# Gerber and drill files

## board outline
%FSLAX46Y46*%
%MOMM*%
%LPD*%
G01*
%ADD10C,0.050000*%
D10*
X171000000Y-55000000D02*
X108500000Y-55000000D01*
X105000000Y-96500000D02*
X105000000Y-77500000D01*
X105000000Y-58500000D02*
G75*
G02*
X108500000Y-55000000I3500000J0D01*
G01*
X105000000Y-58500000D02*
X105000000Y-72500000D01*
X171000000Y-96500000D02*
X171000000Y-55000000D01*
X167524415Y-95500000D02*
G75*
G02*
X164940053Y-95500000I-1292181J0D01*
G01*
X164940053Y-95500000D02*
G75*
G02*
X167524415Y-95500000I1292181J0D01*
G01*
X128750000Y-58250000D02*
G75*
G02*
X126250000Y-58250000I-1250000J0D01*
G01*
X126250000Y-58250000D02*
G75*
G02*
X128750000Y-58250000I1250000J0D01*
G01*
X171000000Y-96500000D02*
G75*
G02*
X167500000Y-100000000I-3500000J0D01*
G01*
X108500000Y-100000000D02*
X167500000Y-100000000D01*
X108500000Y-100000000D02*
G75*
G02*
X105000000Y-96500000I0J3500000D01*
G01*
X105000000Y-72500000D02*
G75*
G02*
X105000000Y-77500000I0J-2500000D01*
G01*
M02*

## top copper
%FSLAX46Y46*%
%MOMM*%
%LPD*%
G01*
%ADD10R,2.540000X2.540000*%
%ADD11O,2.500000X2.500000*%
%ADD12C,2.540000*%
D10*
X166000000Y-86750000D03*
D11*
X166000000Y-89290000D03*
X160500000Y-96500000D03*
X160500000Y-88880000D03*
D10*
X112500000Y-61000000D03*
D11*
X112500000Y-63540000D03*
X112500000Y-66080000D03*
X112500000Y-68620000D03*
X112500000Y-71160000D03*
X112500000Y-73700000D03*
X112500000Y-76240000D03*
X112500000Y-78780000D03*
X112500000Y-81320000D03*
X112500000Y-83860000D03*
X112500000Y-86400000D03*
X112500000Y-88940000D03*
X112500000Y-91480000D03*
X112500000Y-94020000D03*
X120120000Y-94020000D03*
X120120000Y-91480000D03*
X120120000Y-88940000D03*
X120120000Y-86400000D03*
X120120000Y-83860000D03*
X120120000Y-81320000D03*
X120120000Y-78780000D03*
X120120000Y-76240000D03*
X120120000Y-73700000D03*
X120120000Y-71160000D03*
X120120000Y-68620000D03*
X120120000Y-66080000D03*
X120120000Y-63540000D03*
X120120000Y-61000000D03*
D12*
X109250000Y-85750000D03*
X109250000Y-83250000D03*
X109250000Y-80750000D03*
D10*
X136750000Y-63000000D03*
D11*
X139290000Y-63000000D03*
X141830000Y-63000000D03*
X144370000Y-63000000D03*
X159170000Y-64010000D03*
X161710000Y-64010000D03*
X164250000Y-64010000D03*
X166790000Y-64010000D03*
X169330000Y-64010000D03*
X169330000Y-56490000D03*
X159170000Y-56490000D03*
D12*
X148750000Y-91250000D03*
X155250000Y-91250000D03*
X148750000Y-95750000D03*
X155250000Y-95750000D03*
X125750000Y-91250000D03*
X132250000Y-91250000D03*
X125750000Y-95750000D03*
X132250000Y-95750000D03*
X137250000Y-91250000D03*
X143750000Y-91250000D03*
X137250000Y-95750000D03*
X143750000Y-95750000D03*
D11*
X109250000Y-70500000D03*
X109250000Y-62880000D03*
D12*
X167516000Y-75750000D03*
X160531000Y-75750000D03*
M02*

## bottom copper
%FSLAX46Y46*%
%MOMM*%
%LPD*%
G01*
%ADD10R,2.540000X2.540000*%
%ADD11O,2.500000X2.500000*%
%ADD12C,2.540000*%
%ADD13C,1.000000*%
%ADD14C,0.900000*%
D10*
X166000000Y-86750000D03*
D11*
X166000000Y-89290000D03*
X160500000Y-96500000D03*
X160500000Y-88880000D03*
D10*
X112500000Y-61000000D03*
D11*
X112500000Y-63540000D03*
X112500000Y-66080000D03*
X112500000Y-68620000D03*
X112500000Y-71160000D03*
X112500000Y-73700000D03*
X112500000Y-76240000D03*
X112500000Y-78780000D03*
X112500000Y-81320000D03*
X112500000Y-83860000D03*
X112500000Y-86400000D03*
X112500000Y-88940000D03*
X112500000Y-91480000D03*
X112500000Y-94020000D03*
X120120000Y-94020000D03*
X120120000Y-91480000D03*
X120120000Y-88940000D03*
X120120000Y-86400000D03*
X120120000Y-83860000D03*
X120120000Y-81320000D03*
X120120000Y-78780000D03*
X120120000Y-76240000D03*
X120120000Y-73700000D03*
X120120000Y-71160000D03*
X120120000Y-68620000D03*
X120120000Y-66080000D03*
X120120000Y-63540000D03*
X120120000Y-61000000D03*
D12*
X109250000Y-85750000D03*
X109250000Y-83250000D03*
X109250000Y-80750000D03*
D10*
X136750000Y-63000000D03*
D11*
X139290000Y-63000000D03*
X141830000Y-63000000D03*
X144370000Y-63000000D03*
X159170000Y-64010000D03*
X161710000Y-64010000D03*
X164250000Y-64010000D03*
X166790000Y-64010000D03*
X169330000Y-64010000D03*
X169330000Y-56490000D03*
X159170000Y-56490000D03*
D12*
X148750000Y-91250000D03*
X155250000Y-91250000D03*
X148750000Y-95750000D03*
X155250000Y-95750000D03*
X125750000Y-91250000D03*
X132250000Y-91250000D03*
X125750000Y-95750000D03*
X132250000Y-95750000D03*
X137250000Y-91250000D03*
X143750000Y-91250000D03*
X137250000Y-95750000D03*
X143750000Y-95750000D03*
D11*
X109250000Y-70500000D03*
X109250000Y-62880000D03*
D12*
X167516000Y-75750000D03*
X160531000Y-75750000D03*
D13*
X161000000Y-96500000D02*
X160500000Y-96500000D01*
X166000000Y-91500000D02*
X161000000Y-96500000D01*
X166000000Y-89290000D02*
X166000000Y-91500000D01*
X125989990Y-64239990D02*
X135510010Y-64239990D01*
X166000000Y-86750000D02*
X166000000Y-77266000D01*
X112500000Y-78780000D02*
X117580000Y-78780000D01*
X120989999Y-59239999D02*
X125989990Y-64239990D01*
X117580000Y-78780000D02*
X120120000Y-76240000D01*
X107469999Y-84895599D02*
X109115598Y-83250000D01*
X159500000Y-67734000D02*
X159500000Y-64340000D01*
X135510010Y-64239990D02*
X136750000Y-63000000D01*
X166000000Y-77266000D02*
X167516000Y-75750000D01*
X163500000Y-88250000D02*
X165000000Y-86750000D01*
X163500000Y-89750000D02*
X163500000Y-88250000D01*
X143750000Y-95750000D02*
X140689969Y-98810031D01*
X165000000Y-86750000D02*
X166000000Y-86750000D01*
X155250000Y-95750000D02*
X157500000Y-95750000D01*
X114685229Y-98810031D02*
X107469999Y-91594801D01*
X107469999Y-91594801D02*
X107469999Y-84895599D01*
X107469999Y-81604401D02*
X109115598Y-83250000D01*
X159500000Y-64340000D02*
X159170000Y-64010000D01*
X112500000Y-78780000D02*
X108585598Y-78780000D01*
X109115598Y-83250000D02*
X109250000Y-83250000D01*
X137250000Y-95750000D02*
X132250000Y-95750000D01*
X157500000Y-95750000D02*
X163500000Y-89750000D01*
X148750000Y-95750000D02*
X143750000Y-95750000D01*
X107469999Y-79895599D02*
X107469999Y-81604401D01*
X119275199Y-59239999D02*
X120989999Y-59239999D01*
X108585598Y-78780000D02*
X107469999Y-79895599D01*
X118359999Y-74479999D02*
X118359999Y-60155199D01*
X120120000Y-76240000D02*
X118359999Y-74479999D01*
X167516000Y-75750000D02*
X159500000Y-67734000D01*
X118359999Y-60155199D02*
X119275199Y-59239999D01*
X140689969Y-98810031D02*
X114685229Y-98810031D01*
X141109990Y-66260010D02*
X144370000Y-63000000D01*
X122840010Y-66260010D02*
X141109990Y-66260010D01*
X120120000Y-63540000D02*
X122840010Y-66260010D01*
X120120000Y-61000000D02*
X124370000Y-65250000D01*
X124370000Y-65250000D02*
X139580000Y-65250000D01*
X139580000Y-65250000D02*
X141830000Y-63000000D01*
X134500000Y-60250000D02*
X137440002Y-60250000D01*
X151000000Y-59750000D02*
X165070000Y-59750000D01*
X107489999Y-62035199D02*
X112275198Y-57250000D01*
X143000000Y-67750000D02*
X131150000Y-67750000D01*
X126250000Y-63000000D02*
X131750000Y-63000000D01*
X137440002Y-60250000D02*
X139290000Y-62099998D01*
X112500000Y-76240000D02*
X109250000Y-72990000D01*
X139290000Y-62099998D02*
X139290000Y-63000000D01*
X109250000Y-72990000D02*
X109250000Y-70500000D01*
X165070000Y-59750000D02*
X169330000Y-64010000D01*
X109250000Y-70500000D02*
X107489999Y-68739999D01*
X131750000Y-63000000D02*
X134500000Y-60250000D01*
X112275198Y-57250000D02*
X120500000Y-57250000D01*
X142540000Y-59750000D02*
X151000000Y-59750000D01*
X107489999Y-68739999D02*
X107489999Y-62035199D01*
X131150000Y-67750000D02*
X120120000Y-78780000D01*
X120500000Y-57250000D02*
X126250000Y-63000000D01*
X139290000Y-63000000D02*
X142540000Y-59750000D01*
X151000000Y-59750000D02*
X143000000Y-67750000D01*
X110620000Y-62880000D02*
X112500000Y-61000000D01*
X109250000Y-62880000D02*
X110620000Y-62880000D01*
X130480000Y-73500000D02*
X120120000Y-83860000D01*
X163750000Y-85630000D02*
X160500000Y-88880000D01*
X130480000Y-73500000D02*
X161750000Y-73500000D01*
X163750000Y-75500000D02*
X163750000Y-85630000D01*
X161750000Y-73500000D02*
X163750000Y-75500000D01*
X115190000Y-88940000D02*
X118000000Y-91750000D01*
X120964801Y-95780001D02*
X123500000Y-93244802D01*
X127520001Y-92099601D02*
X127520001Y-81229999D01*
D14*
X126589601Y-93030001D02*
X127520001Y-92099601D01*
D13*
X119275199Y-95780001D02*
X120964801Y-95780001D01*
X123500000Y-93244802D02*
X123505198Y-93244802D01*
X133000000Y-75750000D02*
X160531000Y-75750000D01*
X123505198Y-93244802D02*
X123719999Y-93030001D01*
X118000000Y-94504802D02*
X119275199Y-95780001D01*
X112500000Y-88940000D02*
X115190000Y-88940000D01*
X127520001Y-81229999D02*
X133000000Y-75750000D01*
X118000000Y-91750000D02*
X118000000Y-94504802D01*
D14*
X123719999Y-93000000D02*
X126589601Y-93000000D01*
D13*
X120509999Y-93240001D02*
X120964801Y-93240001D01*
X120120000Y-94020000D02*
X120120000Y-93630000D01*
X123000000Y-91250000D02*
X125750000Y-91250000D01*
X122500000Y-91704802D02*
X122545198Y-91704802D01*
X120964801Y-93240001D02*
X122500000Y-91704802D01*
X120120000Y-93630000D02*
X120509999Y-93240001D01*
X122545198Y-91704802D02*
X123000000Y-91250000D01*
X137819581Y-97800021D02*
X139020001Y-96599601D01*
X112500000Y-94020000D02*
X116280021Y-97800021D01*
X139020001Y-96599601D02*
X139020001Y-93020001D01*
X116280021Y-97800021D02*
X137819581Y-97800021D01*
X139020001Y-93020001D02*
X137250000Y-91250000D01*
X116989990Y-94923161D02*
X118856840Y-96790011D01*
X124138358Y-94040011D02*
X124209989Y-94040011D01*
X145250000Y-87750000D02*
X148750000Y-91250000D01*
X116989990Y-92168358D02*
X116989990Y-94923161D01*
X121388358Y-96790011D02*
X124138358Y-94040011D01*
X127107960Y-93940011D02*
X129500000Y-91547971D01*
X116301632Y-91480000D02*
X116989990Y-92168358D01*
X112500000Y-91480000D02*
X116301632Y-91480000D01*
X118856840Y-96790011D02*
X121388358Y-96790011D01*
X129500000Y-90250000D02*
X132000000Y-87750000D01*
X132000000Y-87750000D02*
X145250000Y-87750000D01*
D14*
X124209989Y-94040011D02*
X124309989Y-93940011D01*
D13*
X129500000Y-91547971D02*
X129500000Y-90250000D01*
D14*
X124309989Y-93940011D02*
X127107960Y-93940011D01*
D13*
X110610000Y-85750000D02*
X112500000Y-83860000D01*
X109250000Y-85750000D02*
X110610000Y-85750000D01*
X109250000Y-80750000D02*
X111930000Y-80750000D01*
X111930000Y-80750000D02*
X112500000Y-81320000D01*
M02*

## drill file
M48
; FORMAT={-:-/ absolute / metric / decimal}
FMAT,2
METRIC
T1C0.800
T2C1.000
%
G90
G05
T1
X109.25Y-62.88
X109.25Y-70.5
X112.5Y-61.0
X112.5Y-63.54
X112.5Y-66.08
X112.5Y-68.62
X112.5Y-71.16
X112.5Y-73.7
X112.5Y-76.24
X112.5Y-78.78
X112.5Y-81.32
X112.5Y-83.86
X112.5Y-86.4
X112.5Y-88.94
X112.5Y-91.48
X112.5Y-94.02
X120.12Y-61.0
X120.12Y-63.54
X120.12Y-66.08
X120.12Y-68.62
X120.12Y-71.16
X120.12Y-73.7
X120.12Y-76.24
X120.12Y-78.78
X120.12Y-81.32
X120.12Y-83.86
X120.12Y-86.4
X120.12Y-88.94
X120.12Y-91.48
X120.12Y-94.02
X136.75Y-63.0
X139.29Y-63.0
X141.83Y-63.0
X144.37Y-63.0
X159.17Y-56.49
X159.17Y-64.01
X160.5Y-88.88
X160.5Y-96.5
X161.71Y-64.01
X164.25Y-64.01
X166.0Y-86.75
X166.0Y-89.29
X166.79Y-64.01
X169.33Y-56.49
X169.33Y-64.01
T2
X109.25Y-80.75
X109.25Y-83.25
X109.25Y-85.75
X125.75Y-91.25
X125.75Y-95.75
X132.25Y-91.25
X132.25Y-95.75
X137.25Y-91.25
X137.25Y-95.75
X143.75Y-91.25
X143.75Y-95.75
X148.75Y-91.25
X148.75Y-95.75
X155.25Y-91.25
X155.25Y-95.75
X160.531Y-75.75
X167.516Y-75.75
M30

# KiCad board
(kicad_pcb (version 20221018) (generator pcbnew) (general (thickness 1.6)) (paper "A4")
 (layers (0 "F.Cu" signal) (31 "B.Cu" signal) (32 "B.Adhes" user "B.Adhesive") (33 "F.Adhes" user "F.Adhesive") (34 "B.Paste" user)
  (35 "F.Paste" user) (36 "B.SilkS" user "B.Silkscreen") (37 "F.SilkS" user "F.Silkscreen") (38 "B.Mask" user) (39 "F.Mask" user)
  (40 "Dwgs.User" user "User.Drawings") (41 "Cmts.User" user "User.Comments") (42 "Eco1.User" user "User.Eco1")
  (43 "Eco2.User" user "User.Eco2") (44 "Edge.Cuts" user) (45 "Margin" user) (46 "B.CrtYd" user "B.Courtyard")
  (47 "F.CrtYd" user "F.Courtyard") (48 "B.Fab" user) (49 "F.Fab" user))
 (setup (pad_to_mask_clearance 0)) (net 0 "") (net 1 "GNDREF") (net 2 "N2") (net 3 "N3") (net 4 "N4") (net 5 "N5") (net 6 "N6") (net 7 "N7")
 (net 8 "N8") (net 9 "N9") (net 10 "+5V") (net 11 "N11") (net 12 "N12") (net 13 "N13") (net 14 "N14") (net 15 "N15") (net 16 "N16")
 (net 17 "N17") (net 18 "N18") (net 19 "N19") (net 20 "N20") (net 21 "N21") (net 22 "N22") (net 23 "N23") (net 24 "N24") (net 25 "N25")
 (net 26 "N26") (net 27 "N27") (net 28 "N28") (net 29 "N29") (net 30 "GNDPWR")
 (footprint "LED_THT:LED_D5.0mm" (layer "F.Cu") (at 166 86.75 -90)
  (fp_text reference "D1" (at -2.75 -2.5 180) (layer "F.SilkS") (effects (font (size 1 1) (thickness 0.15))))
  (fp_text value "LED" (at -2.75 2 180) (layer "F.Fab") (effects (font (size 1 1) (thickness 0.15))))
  (pad "1" thru_hole rect (at 0 0 270) (size 2.54 2.54) (drill 0.8) (layers "*.Cu" "*.Mask") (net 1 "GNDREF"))
  (pad "2" thru_hole oval (at 2.54 0 270) (size 2.5 2.5) (drill 0.8) (layers "*.Cu" "*.Mask") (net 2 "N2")))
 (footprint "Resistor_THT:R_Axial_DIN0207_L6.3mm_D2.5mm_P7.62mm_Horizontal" (layer "F.Cu") (at 160.5 96.5 90)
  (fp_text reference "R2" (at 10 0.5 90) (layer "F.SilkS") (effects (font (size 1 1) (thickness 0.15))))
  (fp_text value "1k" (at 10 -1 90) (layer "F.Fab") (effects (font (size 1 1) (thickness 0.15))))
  (pad "1" thru_hole oval (at 0 0 90) (size 2.5 2.5) (drill 0.8) (layers "*.Cu" "*.Mask") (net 2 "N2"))
  (pad "2" thru_hole oval (at 7.62 0 90) (size 2.5 2.5) (drill 0.8) (layers "*.Cu" "*.Mask") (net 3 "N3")))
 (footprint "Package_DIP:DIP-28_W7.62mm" (layer "F.Cu") (at 112.5 61)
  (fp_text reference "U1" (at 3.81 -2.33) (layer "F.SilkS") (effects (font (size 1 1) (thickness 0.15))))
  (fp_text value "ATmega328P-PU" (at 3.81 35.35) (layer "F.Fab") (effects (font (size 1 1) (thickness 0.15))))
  (pad "1" thru_hole rect (at 0 0) (size 2.54 2.54) (drill 0.8) (layers "*.Cu" "*.Mask") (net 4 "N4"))
  (pad "2" thru_hole oval (at 0 2.54) (size 2.5 2.5) (drill 0.8) (layers "*.Cu" "*.Mask") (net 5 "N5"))
  (pad "3" thru_hole oval (at 0 5.08) (size 2.5 2.5) (drill 0.8) (layers "*.Cu" "*.Mask") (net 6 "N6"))
  (pad "4" thru_hole oval (at 0 7.62) (size 2.5 2.5) (drill 0.8) (layers "*.Cu" "*.Mask") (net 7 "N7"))
  (pad "5" thru_hole oval (at 0 10.16) (size 2.5 2.5) (drill 0.8) (layers "*.Cu" "*.Mask") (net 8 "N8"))
  (pad "6" thru_hole oval (at 0 12.7) (size 2.5 2.5) (drill 0.8) (layers "*.Cu" "*.Mask") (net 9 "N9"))
  (pad "7" thru_hole oval (at 0 15.24) (size 2.5 2.5) (drill 0.8) (layers "*.Cu" "*.Mask") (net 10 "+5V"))
  (pad "8" thru_hole oval (at 0 17.78) (size 2.5 2.5) (drill 0.8) (layers "*.Cu" "*.Mask") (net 1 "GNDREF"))
  (pad "9" thru_hole oval (at 0 20.32) (size 2.5 2.5) (drill 0.8) (layers "*.Cu" "*.Mask") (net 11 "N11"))
  (pad "10" thru_hole oval (at 0 22.86) (size 2.5 2.5) (drill 0.8) (layers "*.Cu" "*.Mask") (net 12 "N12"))
  (pad "11" thru_hole oval (at 0 25.4) (size 2.5 2.5) (drill 0.8) (layers "*.Cu" "*.Mask") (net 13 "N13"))
  (pad "12" thru_hole oval (at 0 27.94) (size 2.5 2.5) (drill 0.8) (layers "*.Cu" "*.Mask") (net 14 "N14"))
  (pad "13" thru_hole oval (at 0 30.48) (size 2.5 2.5) (drill 0.8) (layers "*.Cu" "*.Mask") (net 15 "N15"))
  (pad "14" thru_hole oval (at 0 33.02) (size 2.5 2.5) (drill 0.8) (layers "*.Cu" "*.Mask") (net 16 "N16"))
  (pad "15" thru_hole oval (at 7.62 33.02) (size 2.5 2.5) (drill 0.8) (layers "*.Cu" "*.Mask") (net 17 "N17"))
  (pad "16" thru_hole oval (at 7.62 30.48) (size 2.5 2.5) (drill 0.8) (layers "*.Cu" "*.Mask") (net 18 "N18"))
  (pad "17" thru_hole oval (at 7.62 27.94) (size 2.5 2.5) (drill 0.8) (layers "*.Cu" "*.Mask") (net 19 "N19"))
  (pad "18" thru_hole oval (at 7.62 25.4) (size 2.5 2.5) (drill 0.8) (layers "*.Cu" "*.Mask") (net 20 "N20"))
  (pad "19" thru_hole oval (at 7.62 22.86) (size 2.5 2.5) (drill 0.8) (layers "*.Cu" "*.Mask") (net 3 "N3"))
  (pad "20" thru_hole oval (at 7.62 20.32) (size 2.5 2.5) (drill 0.8) (layers "*.Cu" "*.Mask") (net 10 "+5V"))
  (pad "21" thru_hole oval (at 7.62 17.78) (size 2.5 2.5) (drill 0.8) (layers "*.Cu" "*.Mask") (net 10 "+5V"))
  (pad "22" thru_hole oval (at 7.62 15.24) (size 2.5 2.5) (drill 0.8) (layers "*.Cu" "*.Mask") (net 1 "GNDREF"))
  (pad "23" thru_hole oval (at 7.62 12.7) (size 2.5 2.5) (drill 0.8) (layers "*.Cu" "*.Mask") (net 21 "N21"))
  (pad "24" thru_hole oval (at 7.62 10.16) (size 2.5 2.5) (drill 0.8) (layers "*.Cu" "*.Mask") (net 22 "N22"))
  (pad "25" thru_hole oval (at 7.62 7.62) (size 2.5 2.5) (drill 0.8) (layers "*.Cu" "*.Mask") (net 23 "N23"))
  (pad "26" thru_hole oval (at 7.62 5.08) (size 2.5 2.5) (drill 0.8) (layers "*.Cu" "*.Mask") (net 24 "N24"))
  (pad "27" thru_hole oval (at 7.62 2.54) (size 2.5 2.5) (drill 0.8) (layers "*.Cu" "*.Mask") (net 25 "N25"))
  (pad "28" thru_hole oval (at 7.62 0) (size 2.5 2.5) (drill 0.8) (layers "*.Cu" "*.Mask") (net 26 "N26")))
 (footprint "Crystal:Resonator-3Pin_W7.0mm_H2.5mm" (layer "F.Cu") (at 109.25 85.75 90)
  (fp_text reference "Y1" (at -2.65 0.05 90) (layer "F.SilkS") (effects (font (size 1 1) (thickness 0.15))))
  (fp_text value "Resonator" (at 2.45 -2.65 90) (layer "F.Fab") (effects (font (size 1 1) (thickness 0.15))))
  (pad "1" thru_hole circle (at 0 0 90) (size 2.54 2.54) (drill 1) (layers "*.Cu" "*.Mask") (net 12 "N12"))
  (pad "2" thru_hole circle (at 2.5 0 90) (size 2.54 2.54) (drill 1) (layers "*.Cu" "*.Mask") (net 1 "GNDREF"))
  (pad "3" thru_hole circle (at 5 0 90) (size 2.54 2.54) (drill 1) (layers "*.Cu" "*.Mask") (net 11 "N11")))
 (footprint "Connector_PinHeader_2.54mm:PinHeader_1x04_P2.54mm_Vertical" (layer "F.Cu") (at 136.75 63 90)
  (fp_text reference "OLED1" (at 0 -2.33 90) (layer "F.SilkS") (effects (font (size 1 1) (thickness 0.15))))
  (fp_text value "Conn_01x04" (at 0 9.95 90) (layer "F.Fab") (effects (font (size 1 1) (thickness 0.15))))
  (pad "1" thru_hole rect (at 0 0 90) (size 2.54 2.54) (drill 0.8) (layers "*.Cu" "*.Mask") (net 1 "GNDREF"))
  (pad "2" thru_hole oval (at 0 2.54 90) (size 2.5 2.5) (drill 0.8) (layers "*.Cu" "*.Mask") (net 10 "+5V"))
  (pad "3" thru_hole oval (at 0 5.08 90) (size 2.5 2.5) (drill 0.8) (layers "*.Cu" "*.Mask") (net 26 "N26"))
  (pad "4" thru_hole oval (at 0 7.62 90) (size 2.5 2.5) (drill 0.8) (layers "*.Cu" "*.Mask") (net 25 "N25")))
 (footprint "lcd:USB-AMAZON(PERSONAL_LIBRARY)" (layer "F.Cu") (at 164.25 60.25)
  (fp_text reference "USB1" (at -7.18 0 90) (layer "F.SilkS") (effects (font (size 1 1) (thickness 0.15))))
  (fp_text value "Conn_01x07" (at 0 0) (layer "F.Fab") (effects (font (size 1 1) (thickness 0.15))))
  (pad "1" thru_hole oval (at -5.08 3.76) (size 2.5 2.5) (drill 0.8) (layers "*.Cu" "*.Mask") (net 1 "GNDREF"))
  (pad "2" thru_hole oval (at -2.54 3.76) (size 2.5 2.5) (drill 0.8) (layers "*.Cu" "*.Mask") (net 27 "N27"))
  (pad "3" thru_hole oval (at 0 3.76) (size 2.5 2.5) (drill 0.8) (layers "*.Cu" "*.Mask") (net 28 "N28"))
  (pad "4" thru_hole oval (at 2.54 3.76) (size 2.5 2.5) (drill 0.8) (layers "*.Cu" "*.Mask") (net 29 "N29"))
  (pad "5" thru_hole oval (at 5.08 3.76) (size 2.5 2.5) (drill 0.8) (layers "*.Cu" "*.Mask") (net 10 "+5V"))
  (pad "6" thru_hole oval (at 5.08 -3.76) (size 2.5 2.5) (drill 0.8) (layers "*.Cu" "*.Mask") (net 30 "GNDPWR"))
  (pad "7" thru_hole oval (at -5.08 -3.76) (size 2.5 2.5) (drill 0.8) (layers "*.Cu" "*.Mask") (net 30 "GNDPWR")))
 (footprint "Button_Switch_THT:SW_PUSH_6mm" (layer "F.Cu") (at 148.75 91.25)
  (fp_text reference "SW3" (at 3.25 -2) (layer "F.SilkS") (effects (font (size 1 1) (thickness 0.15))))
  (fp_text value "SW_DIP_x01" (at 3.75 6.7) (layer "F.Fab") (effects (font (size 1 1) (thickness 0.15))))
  (pad "1" thru_hole circle (at 0 0) (size 2.54 2.54) (drill 1) (layers "*.Cu" "*.Mask") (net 15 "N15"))
  (pad "1" thru_hole circle (at 6.5 0) (size 2.54 2.54) (drill 1) (layers "*.Cu" "*.Mask") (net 15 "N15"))
  (pad "2" thru_hole circle (at 0 4.5) (size 2.54 2.54) (drill 1) (layers "*.Cu" "*.Mask") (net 1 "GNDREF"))
  (pad "2" thru_hole circle (at 6.5 4.5) (size 2.54 2.54) (drill 1) (layers "*.Cu" "*.Mask") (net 1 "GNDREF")))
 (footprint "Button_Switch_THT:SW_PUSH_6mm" (layer "F.Cu") (at 125.75 91.25)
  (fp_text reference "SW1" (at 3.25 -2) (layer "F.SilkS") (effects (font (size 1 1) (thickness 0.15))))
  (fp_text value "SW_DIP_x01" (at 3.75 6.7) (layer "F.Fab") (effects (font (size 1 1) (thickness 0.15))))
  (pad "1" thru_hole circle (at 0 0) (size 2.54 2.54) (drill 1) (layers "*.Cu" "*.Mask") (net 17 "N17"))
  (pad "1" thru_hole circle (at 6.5 0) (size 2.54 2.54) (drill 1) (layers "*.Cu" "*.Mask") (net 17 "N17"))
  (pad "2" thru_hole circle (at 0 4.5) (size 2.54 2.54) (drill 1) (layers "*.Cu" "*.Mask") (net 1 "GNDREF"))
  (pad "2" thru_hole circle (at 6.5 4.5) (size 2.54 2.54) (drill 1) (layers "*.Cu" "*.Mask") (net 1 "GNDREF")))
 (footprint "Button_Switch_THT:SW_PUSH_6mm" (layer "F.Cu") (at 137.25 91.25)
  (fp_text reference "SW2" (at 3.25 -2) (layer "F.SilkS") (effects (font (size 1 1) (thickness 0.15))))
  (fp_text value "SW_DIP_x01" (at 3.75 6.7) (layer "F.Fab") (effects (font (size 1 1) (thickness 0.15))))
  (pad "1" thru_hole circle (at 0 0) (size 2.54 2.54) (drill 1) (layers "*.Cu" "*.Mask") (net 16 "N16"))
  (pad "1" thru_hole circle (at 6.5 0) (size 2.54 2.54) (drill 1) (layers "*.Cu" "*.Mask") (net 16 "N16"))
  (pad "2" thru_hole circle (at 0 4.5) (size 2.54 2.54) (drill 1) (layers "*.Cu" "*.Mask") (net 1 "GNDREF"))
  (pad "2" thru_hole circle (at 6.5 4.5) (size 2.54 2.54) (drill 1) (layers "*.Cu" "*.Mask") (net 1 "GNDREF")))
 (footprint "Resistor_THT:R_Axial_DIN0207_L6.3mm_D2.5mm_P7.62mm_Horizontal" (layer "F.Cu") (at 109.25 70.5 90)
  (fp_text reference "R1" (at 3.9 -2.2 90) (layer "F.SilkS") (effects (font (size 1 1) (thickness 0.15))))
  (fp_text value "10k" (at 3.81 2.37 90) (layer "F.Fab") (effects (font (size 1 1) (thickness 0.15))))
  (pad "1" thru_hole oval (at 0 0 90) (size 2.5 2.5) (drill 0.8) (layers "*.Cu" "*.Mask") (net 10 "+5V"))
  (pad "2" thru_hole oval (at 7.62 0 90) (size 2.5 2.5) (drill 0.8) (layers "*.Cu" "*.Mask") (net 4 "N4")))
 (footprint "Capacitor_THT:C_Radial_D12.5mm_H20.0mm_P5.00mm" (layer "F.Cu") (at 166.5 75.75 180)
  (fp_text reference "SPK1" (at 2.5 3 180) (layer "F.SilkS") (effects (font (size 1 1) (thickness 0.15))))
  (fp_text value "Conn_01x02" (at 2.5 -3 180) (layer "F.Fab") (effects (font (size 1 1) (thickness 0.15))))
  (pad "1" thru_hole circle (at -1.016 0 180) (size 2.54 2.54) (drill 1) (layers "*.Cu" "*.Mask") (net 1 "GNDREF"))
  (pad "2" thru_hole circle (at 5.969 0 180) (size 2.54 2.54) (drill 1) (layers "*.Cu" "*.Mask") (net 14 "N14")))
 (gr_line (start 171 55) (end 108.5 55) (stroke (width 0.05) (type solid)) (layer "Edge.Cuts"))
 (gr_line (start 105 96.5) (end 105 77.5) (stroke (width 0.05) (type solid)) (layer "Edge.Cuts"))
 (gr_arc (start 105 58.5) (mid 106.025126 56.025126) (end 108.5 55) (stroke (width 0.05) (type solid)) (layer "Edge.Cuts"))
 (gr_line (start 105 58.5) (end 105 72.5) (stroke (width 0.05) (type solid)) (layer "Edge.Cuts"))
 (gr_line (start 171 96.5) (end 171 55) (stroke (width 0.05) (type solid)) (layer "Edge.Cuts"))
 (gr_circle (center 166.232234 95.5) (end 167.5 95.25) (stroke (width 0.05) (type solid)) (fill none) (layer "Edge.Cuts"))
 (gr_circle (center 127.5 58.25) (end 128.75 58.25) (stroke (width 0.05) (type solid)) (fill none) (layer "Edge.Cuts"))
 (gr_arc (start 171 96.5) (mid 169.974874 98.974874) (end 167.5 100) (stroke (width 0.05) (type solid)) (layer "Edge.Cuts"))
 (gr_line (start 108.5 100) (end 167.5 100) (stroke (width 0.05) (type solid)) (layer "Edge.Cuts"))
 (gr_arc (start 108.5 100) (mid 106.025126 98.974874) (end 105 96.5) (stroke (width 0.05) (type solid)) (layer "Edge.Cuts"))
 (gr_arc (start 105 72.5) (mid 107.5 75) (end 105 77.5) (stroke (width 0.05) (type solid)) (layer "Edge.Cuts"))
 (segment (start 161 96.5) (end 160.5 96.5) (width 1) (layer "B.Cu") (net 2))
 (segment (start 166 91.5) (end 161 96.5) (width 1) (layer "B.Cu") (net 2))
 (segment (start 166 89.29) (end 166 91.5) (width 1) (layer "B.Cu") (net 2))
 (segment (start 125.98999 64.23999) (end 135.51001 64.23999) (width 1) (layer "B.Cu") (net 1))
 (segment (start 166 86.75) (end 166 77.266) (width 1) (layer "B.Cu") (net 1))
 (segment (start 112.5 78.78) (end 117.58 78.78) (width 1) (layer "B.Cu") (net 1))
 (segment (start 120.989999 59.239999) (end 125.98999 64.23999) (width 1) (layer "B.Cu") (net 1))
 (segment (start 117.58 78.78) (end 120.12 76.24) (width 1) (layer "B.Cu") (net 1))
 (segment (start 107.469999 84.895599) (end 109.115598 83.25) (width 1) (layer "B.Cu") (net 1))
 (segment (start 159.5 67.734) (end 159.5 64.34) (width 1) (layer "B.Cu") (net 1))
 (segment (start 135.51001 64.23999) (end 136.75 63) (width 1) (layer "B.Cu") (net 1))
 (segment (start 166 77.266) (end 167.516 75.75) (width 1) (layer "B.Cu") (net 1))
 (segment (start 163.5 88.25) (end 165 86.75) (width 1) (layer "B.Cu") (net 1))
 (segment (start 163.5 89.75) (end 163.5 88.25) (width 1) (layer "B.Cu") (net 1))
 (segment (start 143.75 95.75) (end 140.689969 98.810031) (width 1) (layer "B.Cu") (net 1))
 (segment (start 165 86.75) (end 166 86.75) (width 1) (layer "B.Cu") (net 1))
 (segment (start 155.25 95.75) (end 157.5 95.75) (width 1) (layer "B.Cu") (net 1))
 (segment (start 114.685229 98.810031) (end 107.469999 91.594801) (width 1) (layer "B.Cu") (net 1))
 (segment (start 107.469999 91.594801) (end 107.469999 84.895599) (width 1) (layer "B.Cu") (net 1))
 (segment (start 107.469999 81.604401) (end 109.115598 83.25) (width 1) (layer "B.Cu") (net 1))
 (segment (start 159.5 64.34) (end 159.17 64.01) (width 1) (layer "B.Cu") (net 1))
 (segment (start 112.5 78.78) (end 108.585598 78.78) (width 1) (layer "B.Cu") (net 1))
 (segment (start 109.115598 83.25) (end 109.25 83.25) (width 1) (layer "B.Cu") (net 1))
 (segment (start 137.25 95.75) (end 132.25 95.75) (width 1) (layer "B.Cu") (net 1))
 (segment (start 157.5 95.75) (end 163.5 89.75) (width 1) (layer "B.Cu") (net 1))
 (segment (start 148.75 95.75) (end 143.75 95.75) (width 1) (layer "B.Cu") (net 1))
 (segment (start 107.469999 79.895599) (end 107.469999 81.604401) (width 1) (layer "B.Cu") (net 1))
 (segment (start 119.275199 59.239999) (end 120.989999 59.239999) (width 1) (layer "B.Cu") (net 1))
 (segment (start 108.585598 78.78) (end 107.469999 79.895599) (width 1) (layer "B.Cu") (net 1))
 (segment (start 118.359999 74.479999) (end 118.359999 60.155199) (width 1) (layer "B.Cu") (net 1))
 (segment (start 120.12 76.24) (end 118.359999 74.479999) (width 1) (layer "B.Cu") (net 1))
 (segment (start 167.516 75.75) (end 159.5 67.734) (width 1) (layer "B.Cu") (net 1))
 (segment (start 118.359999 60.155199) (end 119.275199 59.239999) (width 1) (layer "B.Cu") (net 1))
 (segment (start 140.689969 98.810031) (end 114.685229 98.810031) (width 1) (layer "B.Cu") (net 1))
 (segment (start 141.10999 66.26001) (end 144.37 63) (width 1) (layer "B.Cu") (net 25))
 (segment (start 122.84001 66.26001) (end 141.10999 66.26001) (width 1) (layer "B.Cu") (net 25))
 (segment (start 120.12 63.54) (end 122.84001 66.26001) (width 1) (layer "B.Cu") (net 25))
 (segment (start 120.12 61) (end 124.37 65.25) (width 1) (layer "B.Cu") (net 26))
 (segment (start 124.37 65.25) (end 139.58 65.25) (width 1) (layer "B.Cu") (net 26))
 (segment (start 139.58 65.25) (end 141.83 63) (width 1) (layer "B.Cu") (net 26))
 (segment (start 134.5 60.25) (end 137.440002 60.25) (width 1) (layer "B.Cu") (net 10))
 (segment (start 151 59.75) (end 165.07 59.75) (width 1) (layer "B.Cu") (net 10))
 (segment (start 107.489999 62.035199) (end 112.275198 57.25) (width 1) (layer "B.Cu") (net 10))
 (segment (start 143 67.75) (end 131.15 67.75) (width 1) (layer "B.Cu") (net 10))
 (segment (start 126.25 63) (end 131.75 63) (width 1) (layer "B.Cu") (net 10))
 (segment (start 137.440002 60.25) (end 139.29 62.099998) (width 1) (layer "B.Cu") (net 10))
 (segment (start 112.5 76.24) (end 109.25 72.99) (width 1) (layer "B.Cu") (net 10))
 (segment (start 139.29 62.099998) (end 139.29 63) (width 1) (layer "B.Cu") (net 10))
 (segment (start 109.25 72.99) (end 109.25 70.5) (width 1) (layer "B.Cu") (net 10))
 (segment (start 165.07 59.75) (end 169.33 64.01) (width 1) (layer "B.Cu") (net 10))
 (segment (start 109.25 70.5) (end 107.489999 68.739999) (width 1) (layer "B.Cu") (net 10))
 (segment (start 131.75 63) (end 134.5 60.25) (width 1) (layer "B.Cu") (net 10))
 (segment (start 112.275198 57.25) (end 120.5 57.25) (width 1) (layer "B.Cu") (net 10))
 (segment (start 142.54 59.75) (end 151 59.75) (width 1) (layer "B.Cu") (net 10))
 (segment (start 107.489999 68.739999) (end 107.489999 62.035199) (width 1) (layer "B.Cu") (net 10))
 (segment (start 131.15 67.75) (end 120.12 78.78) (width 1) (layer "B.Cu") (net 10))
 (segment (start 120.5 57.25) (end 126.25 63) (width 1) (layer "B.Cu") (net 10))
 (segment (start 139.29 63) (end 142.54 59.75) (width 1) (layer "B.Cu") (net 10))
 (segment (start 151 59.75) (end 143 67.75) (width 1) (layer "B.Cu") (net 10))
 (segment (start 110.62 62.88) (end 112.5 61) (width 1) (layer "B.Cu") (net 4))
 (segment (start 109.25 62.88) (end 110.62 62.88) (width 1) (layer "B.Cu") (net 4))
 (segment (start 130.48 73.5) (end 120.12 83.86) (width 1) (layer "B.Cu") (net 3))
 (segment (start 163.75 85.63) (end 160.5 88.88) (width 1) (layer "B.Cu") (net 3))
 (segment (start 130.48 73.5) (end 161.75 73.5) (width 1) (layer "B.Cu") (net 3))
 (segment (start 163.75 75.5) (end 163.75 85.63) (width 1) (layer "B.Cu") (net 3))
 (segment (start 161.75 73.5) (end 163.75 75.5) (width 1) (layer "B.Cu") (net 3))
 (segment (start 115.19 88.94) (end 118 91.75) (width 1) (layer "B.Cu") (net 14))
 (segment (start 120.964801 95.780001) (end 123.5 93.244802) (width 1) (layer "B.Cu") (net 14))
 (segment (start 127.520001 92.099601) (end 127.520001 81.229999) (width 1) (layer "B.Cu") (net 14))
 (segment (start 126.589601 93.030001) (end 127.520001 92.099601) (width 0.9) (layer "B.Cu") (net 14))
 (segment (start 119.275199 95.780001) (end 120.964801 95.780001) (width 1) (layer "B.Cu") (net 14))
 (segment (start 123.5 93.244802) (end 123.505198 93.244802) (width 1) (layer "B.Cu") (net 14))
 (segment (start 133 75.75) (end 160.531 75.75) (width 1) (layer "B.Cu") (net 14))
 (segment (start 123.505198 93.244802) (end 123.719999 93.030001) (width 1) (layer "B.Cu") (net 14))
 (segment (start 118 94.504802) (end 119.275199 95.780001) (width 1) (layer "B.Cu") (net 14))
 (segment (start 112.5 88.94) (end 115.19 88.94) (width 1) (layer "B.Cu") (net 14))
 (segment (start 127.520001 81.229999) (end 133 75.75) (width 1) (layer "B.Cu") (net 14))
 (segment (start 118 91.75) (end 118 94.504802) (width 1) (layer "B.Cu") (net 14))
 (segment (start 123.719999 93) (end 126.589601 93) (width 0.9) (layer "B.Cu") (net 14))
 (segment (start 120.509999 93.240001) (end 120.964801 93.240001) (width 1) (layer "B.Cu") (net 17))
 (segment (start 120.12 94.02) (end 120.12 93.63) (width 1) (layer "B.Cu") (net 17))
 (segment (start 123 91.25) (end 125.75 91.25) (width 1) (layer "B.Cu") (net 17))
 (segment (start 122.5 91.704802) (end 122.545198 91.704802) (width 1) (layer "B.Cu") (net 17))
 (segment (start 120.964801 93.240001) (end 122.5 91.704802) (width 1) (layer "B.Cu") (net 17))
 (segment (start 120.12 93.63) (end 120.509999 93.240001) (width 1) (layer "B.Cu") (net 17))
 (segment (start 122.545198 91.704802) (end 123 91.25) (width 1) (layer "B.Cu") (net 17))
 (segment (start 137.819581 97.800021) (end 139.020001 96.599601) (width 1) (layer "B.Cu") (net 16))
 (segment (start 112.5 94.02) (end 116.280021 97.800021) (width 1) (layer "B.Cu") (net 16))
 (segment (start 139.020001 96.599601) (end 139.020001 93.020001) (width 1) (layer "B.Cu") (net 16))
 (segment (start 116.280021 97.800021) (end 137.819581 97.800021) (width 1) (layer "B.Cu") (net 16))
 (segment (start 139.020001 93.020001) (end 137.25 91.25) (width 1) (layer "B.Cu") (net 16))
 (segment (start 116.98999 94.923161) (end 118.85684 96.790011) (width 1) (layer "B.Cu") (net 15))
 (segment (start 124.138358 94.040011) (end 124.209989 94.040011) (width 1) (layer "B.Cu") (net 15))
 (segment (start 145.25 87.75) (end 148.75 91.25) (width 1) (layer "B.Cu") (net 15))
 (segment (start 116.98999 92.168358) (end 116.98999 94.923161) (width 1) (layer "B.Cu") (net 15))
 (segment (start 121.388358 96.790011) (end 124.138358 94.040011) (width 1) (layer "B.Cu") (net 15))
 (segment (start 127.10796 93.940011) (end 129.5 91.547971) (width 1) (layer "B.Cu") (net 15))
 (segment (start 116.301632 91.48) (end 116.98999 92.168358) (width 1) (layer "B.Cu") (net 15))
 (segment (start 112.5 91.48) (end 116.301632 91.48) (width 1) (layer "B.Cu") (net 15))
 (segment (start 118.85684 96.790011) (end 121.388358 96.790011) (width 1) (layer "B.Cu") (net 15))
 (segment (start 129.5 90.25) (end 132 87.75) (width 1) (layer "B.Cu") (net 15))
 (segment (start 132 87.75) (end 145.25 87.75) (width 1) (layer "B.Cu") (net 15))
 (segment (start 124.209989 94.040011) (end 124.309989 93.940011) (width 0.9) (layer "B.Cu") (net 15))
 (segment (start 129.5 91.547971) (end 129.5 90.25) (width 1) (layer "B.Cu") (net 15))
 (segment (start 124.309989 93.940011) (end 127.10796 93.940011) (width 0.9) (layer "B.Cu") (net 15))
 (segment (start 110.61 85.75) (end 112.5 83.86) (width 1) (layer "B.Cu") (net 12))
 (segment (start 109.25 85.75) (end 110.61 85.75) (width 1) (layer "B.Cu") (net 12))
 (segment (start 109.25 80.75) (end 111.93 80.75) (width 1) (layer "B.Cu") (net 11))
 (segment (start 111.93 80.75) (end 112.5 81.32) (width 1) (layer "B.Cu") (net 11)))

